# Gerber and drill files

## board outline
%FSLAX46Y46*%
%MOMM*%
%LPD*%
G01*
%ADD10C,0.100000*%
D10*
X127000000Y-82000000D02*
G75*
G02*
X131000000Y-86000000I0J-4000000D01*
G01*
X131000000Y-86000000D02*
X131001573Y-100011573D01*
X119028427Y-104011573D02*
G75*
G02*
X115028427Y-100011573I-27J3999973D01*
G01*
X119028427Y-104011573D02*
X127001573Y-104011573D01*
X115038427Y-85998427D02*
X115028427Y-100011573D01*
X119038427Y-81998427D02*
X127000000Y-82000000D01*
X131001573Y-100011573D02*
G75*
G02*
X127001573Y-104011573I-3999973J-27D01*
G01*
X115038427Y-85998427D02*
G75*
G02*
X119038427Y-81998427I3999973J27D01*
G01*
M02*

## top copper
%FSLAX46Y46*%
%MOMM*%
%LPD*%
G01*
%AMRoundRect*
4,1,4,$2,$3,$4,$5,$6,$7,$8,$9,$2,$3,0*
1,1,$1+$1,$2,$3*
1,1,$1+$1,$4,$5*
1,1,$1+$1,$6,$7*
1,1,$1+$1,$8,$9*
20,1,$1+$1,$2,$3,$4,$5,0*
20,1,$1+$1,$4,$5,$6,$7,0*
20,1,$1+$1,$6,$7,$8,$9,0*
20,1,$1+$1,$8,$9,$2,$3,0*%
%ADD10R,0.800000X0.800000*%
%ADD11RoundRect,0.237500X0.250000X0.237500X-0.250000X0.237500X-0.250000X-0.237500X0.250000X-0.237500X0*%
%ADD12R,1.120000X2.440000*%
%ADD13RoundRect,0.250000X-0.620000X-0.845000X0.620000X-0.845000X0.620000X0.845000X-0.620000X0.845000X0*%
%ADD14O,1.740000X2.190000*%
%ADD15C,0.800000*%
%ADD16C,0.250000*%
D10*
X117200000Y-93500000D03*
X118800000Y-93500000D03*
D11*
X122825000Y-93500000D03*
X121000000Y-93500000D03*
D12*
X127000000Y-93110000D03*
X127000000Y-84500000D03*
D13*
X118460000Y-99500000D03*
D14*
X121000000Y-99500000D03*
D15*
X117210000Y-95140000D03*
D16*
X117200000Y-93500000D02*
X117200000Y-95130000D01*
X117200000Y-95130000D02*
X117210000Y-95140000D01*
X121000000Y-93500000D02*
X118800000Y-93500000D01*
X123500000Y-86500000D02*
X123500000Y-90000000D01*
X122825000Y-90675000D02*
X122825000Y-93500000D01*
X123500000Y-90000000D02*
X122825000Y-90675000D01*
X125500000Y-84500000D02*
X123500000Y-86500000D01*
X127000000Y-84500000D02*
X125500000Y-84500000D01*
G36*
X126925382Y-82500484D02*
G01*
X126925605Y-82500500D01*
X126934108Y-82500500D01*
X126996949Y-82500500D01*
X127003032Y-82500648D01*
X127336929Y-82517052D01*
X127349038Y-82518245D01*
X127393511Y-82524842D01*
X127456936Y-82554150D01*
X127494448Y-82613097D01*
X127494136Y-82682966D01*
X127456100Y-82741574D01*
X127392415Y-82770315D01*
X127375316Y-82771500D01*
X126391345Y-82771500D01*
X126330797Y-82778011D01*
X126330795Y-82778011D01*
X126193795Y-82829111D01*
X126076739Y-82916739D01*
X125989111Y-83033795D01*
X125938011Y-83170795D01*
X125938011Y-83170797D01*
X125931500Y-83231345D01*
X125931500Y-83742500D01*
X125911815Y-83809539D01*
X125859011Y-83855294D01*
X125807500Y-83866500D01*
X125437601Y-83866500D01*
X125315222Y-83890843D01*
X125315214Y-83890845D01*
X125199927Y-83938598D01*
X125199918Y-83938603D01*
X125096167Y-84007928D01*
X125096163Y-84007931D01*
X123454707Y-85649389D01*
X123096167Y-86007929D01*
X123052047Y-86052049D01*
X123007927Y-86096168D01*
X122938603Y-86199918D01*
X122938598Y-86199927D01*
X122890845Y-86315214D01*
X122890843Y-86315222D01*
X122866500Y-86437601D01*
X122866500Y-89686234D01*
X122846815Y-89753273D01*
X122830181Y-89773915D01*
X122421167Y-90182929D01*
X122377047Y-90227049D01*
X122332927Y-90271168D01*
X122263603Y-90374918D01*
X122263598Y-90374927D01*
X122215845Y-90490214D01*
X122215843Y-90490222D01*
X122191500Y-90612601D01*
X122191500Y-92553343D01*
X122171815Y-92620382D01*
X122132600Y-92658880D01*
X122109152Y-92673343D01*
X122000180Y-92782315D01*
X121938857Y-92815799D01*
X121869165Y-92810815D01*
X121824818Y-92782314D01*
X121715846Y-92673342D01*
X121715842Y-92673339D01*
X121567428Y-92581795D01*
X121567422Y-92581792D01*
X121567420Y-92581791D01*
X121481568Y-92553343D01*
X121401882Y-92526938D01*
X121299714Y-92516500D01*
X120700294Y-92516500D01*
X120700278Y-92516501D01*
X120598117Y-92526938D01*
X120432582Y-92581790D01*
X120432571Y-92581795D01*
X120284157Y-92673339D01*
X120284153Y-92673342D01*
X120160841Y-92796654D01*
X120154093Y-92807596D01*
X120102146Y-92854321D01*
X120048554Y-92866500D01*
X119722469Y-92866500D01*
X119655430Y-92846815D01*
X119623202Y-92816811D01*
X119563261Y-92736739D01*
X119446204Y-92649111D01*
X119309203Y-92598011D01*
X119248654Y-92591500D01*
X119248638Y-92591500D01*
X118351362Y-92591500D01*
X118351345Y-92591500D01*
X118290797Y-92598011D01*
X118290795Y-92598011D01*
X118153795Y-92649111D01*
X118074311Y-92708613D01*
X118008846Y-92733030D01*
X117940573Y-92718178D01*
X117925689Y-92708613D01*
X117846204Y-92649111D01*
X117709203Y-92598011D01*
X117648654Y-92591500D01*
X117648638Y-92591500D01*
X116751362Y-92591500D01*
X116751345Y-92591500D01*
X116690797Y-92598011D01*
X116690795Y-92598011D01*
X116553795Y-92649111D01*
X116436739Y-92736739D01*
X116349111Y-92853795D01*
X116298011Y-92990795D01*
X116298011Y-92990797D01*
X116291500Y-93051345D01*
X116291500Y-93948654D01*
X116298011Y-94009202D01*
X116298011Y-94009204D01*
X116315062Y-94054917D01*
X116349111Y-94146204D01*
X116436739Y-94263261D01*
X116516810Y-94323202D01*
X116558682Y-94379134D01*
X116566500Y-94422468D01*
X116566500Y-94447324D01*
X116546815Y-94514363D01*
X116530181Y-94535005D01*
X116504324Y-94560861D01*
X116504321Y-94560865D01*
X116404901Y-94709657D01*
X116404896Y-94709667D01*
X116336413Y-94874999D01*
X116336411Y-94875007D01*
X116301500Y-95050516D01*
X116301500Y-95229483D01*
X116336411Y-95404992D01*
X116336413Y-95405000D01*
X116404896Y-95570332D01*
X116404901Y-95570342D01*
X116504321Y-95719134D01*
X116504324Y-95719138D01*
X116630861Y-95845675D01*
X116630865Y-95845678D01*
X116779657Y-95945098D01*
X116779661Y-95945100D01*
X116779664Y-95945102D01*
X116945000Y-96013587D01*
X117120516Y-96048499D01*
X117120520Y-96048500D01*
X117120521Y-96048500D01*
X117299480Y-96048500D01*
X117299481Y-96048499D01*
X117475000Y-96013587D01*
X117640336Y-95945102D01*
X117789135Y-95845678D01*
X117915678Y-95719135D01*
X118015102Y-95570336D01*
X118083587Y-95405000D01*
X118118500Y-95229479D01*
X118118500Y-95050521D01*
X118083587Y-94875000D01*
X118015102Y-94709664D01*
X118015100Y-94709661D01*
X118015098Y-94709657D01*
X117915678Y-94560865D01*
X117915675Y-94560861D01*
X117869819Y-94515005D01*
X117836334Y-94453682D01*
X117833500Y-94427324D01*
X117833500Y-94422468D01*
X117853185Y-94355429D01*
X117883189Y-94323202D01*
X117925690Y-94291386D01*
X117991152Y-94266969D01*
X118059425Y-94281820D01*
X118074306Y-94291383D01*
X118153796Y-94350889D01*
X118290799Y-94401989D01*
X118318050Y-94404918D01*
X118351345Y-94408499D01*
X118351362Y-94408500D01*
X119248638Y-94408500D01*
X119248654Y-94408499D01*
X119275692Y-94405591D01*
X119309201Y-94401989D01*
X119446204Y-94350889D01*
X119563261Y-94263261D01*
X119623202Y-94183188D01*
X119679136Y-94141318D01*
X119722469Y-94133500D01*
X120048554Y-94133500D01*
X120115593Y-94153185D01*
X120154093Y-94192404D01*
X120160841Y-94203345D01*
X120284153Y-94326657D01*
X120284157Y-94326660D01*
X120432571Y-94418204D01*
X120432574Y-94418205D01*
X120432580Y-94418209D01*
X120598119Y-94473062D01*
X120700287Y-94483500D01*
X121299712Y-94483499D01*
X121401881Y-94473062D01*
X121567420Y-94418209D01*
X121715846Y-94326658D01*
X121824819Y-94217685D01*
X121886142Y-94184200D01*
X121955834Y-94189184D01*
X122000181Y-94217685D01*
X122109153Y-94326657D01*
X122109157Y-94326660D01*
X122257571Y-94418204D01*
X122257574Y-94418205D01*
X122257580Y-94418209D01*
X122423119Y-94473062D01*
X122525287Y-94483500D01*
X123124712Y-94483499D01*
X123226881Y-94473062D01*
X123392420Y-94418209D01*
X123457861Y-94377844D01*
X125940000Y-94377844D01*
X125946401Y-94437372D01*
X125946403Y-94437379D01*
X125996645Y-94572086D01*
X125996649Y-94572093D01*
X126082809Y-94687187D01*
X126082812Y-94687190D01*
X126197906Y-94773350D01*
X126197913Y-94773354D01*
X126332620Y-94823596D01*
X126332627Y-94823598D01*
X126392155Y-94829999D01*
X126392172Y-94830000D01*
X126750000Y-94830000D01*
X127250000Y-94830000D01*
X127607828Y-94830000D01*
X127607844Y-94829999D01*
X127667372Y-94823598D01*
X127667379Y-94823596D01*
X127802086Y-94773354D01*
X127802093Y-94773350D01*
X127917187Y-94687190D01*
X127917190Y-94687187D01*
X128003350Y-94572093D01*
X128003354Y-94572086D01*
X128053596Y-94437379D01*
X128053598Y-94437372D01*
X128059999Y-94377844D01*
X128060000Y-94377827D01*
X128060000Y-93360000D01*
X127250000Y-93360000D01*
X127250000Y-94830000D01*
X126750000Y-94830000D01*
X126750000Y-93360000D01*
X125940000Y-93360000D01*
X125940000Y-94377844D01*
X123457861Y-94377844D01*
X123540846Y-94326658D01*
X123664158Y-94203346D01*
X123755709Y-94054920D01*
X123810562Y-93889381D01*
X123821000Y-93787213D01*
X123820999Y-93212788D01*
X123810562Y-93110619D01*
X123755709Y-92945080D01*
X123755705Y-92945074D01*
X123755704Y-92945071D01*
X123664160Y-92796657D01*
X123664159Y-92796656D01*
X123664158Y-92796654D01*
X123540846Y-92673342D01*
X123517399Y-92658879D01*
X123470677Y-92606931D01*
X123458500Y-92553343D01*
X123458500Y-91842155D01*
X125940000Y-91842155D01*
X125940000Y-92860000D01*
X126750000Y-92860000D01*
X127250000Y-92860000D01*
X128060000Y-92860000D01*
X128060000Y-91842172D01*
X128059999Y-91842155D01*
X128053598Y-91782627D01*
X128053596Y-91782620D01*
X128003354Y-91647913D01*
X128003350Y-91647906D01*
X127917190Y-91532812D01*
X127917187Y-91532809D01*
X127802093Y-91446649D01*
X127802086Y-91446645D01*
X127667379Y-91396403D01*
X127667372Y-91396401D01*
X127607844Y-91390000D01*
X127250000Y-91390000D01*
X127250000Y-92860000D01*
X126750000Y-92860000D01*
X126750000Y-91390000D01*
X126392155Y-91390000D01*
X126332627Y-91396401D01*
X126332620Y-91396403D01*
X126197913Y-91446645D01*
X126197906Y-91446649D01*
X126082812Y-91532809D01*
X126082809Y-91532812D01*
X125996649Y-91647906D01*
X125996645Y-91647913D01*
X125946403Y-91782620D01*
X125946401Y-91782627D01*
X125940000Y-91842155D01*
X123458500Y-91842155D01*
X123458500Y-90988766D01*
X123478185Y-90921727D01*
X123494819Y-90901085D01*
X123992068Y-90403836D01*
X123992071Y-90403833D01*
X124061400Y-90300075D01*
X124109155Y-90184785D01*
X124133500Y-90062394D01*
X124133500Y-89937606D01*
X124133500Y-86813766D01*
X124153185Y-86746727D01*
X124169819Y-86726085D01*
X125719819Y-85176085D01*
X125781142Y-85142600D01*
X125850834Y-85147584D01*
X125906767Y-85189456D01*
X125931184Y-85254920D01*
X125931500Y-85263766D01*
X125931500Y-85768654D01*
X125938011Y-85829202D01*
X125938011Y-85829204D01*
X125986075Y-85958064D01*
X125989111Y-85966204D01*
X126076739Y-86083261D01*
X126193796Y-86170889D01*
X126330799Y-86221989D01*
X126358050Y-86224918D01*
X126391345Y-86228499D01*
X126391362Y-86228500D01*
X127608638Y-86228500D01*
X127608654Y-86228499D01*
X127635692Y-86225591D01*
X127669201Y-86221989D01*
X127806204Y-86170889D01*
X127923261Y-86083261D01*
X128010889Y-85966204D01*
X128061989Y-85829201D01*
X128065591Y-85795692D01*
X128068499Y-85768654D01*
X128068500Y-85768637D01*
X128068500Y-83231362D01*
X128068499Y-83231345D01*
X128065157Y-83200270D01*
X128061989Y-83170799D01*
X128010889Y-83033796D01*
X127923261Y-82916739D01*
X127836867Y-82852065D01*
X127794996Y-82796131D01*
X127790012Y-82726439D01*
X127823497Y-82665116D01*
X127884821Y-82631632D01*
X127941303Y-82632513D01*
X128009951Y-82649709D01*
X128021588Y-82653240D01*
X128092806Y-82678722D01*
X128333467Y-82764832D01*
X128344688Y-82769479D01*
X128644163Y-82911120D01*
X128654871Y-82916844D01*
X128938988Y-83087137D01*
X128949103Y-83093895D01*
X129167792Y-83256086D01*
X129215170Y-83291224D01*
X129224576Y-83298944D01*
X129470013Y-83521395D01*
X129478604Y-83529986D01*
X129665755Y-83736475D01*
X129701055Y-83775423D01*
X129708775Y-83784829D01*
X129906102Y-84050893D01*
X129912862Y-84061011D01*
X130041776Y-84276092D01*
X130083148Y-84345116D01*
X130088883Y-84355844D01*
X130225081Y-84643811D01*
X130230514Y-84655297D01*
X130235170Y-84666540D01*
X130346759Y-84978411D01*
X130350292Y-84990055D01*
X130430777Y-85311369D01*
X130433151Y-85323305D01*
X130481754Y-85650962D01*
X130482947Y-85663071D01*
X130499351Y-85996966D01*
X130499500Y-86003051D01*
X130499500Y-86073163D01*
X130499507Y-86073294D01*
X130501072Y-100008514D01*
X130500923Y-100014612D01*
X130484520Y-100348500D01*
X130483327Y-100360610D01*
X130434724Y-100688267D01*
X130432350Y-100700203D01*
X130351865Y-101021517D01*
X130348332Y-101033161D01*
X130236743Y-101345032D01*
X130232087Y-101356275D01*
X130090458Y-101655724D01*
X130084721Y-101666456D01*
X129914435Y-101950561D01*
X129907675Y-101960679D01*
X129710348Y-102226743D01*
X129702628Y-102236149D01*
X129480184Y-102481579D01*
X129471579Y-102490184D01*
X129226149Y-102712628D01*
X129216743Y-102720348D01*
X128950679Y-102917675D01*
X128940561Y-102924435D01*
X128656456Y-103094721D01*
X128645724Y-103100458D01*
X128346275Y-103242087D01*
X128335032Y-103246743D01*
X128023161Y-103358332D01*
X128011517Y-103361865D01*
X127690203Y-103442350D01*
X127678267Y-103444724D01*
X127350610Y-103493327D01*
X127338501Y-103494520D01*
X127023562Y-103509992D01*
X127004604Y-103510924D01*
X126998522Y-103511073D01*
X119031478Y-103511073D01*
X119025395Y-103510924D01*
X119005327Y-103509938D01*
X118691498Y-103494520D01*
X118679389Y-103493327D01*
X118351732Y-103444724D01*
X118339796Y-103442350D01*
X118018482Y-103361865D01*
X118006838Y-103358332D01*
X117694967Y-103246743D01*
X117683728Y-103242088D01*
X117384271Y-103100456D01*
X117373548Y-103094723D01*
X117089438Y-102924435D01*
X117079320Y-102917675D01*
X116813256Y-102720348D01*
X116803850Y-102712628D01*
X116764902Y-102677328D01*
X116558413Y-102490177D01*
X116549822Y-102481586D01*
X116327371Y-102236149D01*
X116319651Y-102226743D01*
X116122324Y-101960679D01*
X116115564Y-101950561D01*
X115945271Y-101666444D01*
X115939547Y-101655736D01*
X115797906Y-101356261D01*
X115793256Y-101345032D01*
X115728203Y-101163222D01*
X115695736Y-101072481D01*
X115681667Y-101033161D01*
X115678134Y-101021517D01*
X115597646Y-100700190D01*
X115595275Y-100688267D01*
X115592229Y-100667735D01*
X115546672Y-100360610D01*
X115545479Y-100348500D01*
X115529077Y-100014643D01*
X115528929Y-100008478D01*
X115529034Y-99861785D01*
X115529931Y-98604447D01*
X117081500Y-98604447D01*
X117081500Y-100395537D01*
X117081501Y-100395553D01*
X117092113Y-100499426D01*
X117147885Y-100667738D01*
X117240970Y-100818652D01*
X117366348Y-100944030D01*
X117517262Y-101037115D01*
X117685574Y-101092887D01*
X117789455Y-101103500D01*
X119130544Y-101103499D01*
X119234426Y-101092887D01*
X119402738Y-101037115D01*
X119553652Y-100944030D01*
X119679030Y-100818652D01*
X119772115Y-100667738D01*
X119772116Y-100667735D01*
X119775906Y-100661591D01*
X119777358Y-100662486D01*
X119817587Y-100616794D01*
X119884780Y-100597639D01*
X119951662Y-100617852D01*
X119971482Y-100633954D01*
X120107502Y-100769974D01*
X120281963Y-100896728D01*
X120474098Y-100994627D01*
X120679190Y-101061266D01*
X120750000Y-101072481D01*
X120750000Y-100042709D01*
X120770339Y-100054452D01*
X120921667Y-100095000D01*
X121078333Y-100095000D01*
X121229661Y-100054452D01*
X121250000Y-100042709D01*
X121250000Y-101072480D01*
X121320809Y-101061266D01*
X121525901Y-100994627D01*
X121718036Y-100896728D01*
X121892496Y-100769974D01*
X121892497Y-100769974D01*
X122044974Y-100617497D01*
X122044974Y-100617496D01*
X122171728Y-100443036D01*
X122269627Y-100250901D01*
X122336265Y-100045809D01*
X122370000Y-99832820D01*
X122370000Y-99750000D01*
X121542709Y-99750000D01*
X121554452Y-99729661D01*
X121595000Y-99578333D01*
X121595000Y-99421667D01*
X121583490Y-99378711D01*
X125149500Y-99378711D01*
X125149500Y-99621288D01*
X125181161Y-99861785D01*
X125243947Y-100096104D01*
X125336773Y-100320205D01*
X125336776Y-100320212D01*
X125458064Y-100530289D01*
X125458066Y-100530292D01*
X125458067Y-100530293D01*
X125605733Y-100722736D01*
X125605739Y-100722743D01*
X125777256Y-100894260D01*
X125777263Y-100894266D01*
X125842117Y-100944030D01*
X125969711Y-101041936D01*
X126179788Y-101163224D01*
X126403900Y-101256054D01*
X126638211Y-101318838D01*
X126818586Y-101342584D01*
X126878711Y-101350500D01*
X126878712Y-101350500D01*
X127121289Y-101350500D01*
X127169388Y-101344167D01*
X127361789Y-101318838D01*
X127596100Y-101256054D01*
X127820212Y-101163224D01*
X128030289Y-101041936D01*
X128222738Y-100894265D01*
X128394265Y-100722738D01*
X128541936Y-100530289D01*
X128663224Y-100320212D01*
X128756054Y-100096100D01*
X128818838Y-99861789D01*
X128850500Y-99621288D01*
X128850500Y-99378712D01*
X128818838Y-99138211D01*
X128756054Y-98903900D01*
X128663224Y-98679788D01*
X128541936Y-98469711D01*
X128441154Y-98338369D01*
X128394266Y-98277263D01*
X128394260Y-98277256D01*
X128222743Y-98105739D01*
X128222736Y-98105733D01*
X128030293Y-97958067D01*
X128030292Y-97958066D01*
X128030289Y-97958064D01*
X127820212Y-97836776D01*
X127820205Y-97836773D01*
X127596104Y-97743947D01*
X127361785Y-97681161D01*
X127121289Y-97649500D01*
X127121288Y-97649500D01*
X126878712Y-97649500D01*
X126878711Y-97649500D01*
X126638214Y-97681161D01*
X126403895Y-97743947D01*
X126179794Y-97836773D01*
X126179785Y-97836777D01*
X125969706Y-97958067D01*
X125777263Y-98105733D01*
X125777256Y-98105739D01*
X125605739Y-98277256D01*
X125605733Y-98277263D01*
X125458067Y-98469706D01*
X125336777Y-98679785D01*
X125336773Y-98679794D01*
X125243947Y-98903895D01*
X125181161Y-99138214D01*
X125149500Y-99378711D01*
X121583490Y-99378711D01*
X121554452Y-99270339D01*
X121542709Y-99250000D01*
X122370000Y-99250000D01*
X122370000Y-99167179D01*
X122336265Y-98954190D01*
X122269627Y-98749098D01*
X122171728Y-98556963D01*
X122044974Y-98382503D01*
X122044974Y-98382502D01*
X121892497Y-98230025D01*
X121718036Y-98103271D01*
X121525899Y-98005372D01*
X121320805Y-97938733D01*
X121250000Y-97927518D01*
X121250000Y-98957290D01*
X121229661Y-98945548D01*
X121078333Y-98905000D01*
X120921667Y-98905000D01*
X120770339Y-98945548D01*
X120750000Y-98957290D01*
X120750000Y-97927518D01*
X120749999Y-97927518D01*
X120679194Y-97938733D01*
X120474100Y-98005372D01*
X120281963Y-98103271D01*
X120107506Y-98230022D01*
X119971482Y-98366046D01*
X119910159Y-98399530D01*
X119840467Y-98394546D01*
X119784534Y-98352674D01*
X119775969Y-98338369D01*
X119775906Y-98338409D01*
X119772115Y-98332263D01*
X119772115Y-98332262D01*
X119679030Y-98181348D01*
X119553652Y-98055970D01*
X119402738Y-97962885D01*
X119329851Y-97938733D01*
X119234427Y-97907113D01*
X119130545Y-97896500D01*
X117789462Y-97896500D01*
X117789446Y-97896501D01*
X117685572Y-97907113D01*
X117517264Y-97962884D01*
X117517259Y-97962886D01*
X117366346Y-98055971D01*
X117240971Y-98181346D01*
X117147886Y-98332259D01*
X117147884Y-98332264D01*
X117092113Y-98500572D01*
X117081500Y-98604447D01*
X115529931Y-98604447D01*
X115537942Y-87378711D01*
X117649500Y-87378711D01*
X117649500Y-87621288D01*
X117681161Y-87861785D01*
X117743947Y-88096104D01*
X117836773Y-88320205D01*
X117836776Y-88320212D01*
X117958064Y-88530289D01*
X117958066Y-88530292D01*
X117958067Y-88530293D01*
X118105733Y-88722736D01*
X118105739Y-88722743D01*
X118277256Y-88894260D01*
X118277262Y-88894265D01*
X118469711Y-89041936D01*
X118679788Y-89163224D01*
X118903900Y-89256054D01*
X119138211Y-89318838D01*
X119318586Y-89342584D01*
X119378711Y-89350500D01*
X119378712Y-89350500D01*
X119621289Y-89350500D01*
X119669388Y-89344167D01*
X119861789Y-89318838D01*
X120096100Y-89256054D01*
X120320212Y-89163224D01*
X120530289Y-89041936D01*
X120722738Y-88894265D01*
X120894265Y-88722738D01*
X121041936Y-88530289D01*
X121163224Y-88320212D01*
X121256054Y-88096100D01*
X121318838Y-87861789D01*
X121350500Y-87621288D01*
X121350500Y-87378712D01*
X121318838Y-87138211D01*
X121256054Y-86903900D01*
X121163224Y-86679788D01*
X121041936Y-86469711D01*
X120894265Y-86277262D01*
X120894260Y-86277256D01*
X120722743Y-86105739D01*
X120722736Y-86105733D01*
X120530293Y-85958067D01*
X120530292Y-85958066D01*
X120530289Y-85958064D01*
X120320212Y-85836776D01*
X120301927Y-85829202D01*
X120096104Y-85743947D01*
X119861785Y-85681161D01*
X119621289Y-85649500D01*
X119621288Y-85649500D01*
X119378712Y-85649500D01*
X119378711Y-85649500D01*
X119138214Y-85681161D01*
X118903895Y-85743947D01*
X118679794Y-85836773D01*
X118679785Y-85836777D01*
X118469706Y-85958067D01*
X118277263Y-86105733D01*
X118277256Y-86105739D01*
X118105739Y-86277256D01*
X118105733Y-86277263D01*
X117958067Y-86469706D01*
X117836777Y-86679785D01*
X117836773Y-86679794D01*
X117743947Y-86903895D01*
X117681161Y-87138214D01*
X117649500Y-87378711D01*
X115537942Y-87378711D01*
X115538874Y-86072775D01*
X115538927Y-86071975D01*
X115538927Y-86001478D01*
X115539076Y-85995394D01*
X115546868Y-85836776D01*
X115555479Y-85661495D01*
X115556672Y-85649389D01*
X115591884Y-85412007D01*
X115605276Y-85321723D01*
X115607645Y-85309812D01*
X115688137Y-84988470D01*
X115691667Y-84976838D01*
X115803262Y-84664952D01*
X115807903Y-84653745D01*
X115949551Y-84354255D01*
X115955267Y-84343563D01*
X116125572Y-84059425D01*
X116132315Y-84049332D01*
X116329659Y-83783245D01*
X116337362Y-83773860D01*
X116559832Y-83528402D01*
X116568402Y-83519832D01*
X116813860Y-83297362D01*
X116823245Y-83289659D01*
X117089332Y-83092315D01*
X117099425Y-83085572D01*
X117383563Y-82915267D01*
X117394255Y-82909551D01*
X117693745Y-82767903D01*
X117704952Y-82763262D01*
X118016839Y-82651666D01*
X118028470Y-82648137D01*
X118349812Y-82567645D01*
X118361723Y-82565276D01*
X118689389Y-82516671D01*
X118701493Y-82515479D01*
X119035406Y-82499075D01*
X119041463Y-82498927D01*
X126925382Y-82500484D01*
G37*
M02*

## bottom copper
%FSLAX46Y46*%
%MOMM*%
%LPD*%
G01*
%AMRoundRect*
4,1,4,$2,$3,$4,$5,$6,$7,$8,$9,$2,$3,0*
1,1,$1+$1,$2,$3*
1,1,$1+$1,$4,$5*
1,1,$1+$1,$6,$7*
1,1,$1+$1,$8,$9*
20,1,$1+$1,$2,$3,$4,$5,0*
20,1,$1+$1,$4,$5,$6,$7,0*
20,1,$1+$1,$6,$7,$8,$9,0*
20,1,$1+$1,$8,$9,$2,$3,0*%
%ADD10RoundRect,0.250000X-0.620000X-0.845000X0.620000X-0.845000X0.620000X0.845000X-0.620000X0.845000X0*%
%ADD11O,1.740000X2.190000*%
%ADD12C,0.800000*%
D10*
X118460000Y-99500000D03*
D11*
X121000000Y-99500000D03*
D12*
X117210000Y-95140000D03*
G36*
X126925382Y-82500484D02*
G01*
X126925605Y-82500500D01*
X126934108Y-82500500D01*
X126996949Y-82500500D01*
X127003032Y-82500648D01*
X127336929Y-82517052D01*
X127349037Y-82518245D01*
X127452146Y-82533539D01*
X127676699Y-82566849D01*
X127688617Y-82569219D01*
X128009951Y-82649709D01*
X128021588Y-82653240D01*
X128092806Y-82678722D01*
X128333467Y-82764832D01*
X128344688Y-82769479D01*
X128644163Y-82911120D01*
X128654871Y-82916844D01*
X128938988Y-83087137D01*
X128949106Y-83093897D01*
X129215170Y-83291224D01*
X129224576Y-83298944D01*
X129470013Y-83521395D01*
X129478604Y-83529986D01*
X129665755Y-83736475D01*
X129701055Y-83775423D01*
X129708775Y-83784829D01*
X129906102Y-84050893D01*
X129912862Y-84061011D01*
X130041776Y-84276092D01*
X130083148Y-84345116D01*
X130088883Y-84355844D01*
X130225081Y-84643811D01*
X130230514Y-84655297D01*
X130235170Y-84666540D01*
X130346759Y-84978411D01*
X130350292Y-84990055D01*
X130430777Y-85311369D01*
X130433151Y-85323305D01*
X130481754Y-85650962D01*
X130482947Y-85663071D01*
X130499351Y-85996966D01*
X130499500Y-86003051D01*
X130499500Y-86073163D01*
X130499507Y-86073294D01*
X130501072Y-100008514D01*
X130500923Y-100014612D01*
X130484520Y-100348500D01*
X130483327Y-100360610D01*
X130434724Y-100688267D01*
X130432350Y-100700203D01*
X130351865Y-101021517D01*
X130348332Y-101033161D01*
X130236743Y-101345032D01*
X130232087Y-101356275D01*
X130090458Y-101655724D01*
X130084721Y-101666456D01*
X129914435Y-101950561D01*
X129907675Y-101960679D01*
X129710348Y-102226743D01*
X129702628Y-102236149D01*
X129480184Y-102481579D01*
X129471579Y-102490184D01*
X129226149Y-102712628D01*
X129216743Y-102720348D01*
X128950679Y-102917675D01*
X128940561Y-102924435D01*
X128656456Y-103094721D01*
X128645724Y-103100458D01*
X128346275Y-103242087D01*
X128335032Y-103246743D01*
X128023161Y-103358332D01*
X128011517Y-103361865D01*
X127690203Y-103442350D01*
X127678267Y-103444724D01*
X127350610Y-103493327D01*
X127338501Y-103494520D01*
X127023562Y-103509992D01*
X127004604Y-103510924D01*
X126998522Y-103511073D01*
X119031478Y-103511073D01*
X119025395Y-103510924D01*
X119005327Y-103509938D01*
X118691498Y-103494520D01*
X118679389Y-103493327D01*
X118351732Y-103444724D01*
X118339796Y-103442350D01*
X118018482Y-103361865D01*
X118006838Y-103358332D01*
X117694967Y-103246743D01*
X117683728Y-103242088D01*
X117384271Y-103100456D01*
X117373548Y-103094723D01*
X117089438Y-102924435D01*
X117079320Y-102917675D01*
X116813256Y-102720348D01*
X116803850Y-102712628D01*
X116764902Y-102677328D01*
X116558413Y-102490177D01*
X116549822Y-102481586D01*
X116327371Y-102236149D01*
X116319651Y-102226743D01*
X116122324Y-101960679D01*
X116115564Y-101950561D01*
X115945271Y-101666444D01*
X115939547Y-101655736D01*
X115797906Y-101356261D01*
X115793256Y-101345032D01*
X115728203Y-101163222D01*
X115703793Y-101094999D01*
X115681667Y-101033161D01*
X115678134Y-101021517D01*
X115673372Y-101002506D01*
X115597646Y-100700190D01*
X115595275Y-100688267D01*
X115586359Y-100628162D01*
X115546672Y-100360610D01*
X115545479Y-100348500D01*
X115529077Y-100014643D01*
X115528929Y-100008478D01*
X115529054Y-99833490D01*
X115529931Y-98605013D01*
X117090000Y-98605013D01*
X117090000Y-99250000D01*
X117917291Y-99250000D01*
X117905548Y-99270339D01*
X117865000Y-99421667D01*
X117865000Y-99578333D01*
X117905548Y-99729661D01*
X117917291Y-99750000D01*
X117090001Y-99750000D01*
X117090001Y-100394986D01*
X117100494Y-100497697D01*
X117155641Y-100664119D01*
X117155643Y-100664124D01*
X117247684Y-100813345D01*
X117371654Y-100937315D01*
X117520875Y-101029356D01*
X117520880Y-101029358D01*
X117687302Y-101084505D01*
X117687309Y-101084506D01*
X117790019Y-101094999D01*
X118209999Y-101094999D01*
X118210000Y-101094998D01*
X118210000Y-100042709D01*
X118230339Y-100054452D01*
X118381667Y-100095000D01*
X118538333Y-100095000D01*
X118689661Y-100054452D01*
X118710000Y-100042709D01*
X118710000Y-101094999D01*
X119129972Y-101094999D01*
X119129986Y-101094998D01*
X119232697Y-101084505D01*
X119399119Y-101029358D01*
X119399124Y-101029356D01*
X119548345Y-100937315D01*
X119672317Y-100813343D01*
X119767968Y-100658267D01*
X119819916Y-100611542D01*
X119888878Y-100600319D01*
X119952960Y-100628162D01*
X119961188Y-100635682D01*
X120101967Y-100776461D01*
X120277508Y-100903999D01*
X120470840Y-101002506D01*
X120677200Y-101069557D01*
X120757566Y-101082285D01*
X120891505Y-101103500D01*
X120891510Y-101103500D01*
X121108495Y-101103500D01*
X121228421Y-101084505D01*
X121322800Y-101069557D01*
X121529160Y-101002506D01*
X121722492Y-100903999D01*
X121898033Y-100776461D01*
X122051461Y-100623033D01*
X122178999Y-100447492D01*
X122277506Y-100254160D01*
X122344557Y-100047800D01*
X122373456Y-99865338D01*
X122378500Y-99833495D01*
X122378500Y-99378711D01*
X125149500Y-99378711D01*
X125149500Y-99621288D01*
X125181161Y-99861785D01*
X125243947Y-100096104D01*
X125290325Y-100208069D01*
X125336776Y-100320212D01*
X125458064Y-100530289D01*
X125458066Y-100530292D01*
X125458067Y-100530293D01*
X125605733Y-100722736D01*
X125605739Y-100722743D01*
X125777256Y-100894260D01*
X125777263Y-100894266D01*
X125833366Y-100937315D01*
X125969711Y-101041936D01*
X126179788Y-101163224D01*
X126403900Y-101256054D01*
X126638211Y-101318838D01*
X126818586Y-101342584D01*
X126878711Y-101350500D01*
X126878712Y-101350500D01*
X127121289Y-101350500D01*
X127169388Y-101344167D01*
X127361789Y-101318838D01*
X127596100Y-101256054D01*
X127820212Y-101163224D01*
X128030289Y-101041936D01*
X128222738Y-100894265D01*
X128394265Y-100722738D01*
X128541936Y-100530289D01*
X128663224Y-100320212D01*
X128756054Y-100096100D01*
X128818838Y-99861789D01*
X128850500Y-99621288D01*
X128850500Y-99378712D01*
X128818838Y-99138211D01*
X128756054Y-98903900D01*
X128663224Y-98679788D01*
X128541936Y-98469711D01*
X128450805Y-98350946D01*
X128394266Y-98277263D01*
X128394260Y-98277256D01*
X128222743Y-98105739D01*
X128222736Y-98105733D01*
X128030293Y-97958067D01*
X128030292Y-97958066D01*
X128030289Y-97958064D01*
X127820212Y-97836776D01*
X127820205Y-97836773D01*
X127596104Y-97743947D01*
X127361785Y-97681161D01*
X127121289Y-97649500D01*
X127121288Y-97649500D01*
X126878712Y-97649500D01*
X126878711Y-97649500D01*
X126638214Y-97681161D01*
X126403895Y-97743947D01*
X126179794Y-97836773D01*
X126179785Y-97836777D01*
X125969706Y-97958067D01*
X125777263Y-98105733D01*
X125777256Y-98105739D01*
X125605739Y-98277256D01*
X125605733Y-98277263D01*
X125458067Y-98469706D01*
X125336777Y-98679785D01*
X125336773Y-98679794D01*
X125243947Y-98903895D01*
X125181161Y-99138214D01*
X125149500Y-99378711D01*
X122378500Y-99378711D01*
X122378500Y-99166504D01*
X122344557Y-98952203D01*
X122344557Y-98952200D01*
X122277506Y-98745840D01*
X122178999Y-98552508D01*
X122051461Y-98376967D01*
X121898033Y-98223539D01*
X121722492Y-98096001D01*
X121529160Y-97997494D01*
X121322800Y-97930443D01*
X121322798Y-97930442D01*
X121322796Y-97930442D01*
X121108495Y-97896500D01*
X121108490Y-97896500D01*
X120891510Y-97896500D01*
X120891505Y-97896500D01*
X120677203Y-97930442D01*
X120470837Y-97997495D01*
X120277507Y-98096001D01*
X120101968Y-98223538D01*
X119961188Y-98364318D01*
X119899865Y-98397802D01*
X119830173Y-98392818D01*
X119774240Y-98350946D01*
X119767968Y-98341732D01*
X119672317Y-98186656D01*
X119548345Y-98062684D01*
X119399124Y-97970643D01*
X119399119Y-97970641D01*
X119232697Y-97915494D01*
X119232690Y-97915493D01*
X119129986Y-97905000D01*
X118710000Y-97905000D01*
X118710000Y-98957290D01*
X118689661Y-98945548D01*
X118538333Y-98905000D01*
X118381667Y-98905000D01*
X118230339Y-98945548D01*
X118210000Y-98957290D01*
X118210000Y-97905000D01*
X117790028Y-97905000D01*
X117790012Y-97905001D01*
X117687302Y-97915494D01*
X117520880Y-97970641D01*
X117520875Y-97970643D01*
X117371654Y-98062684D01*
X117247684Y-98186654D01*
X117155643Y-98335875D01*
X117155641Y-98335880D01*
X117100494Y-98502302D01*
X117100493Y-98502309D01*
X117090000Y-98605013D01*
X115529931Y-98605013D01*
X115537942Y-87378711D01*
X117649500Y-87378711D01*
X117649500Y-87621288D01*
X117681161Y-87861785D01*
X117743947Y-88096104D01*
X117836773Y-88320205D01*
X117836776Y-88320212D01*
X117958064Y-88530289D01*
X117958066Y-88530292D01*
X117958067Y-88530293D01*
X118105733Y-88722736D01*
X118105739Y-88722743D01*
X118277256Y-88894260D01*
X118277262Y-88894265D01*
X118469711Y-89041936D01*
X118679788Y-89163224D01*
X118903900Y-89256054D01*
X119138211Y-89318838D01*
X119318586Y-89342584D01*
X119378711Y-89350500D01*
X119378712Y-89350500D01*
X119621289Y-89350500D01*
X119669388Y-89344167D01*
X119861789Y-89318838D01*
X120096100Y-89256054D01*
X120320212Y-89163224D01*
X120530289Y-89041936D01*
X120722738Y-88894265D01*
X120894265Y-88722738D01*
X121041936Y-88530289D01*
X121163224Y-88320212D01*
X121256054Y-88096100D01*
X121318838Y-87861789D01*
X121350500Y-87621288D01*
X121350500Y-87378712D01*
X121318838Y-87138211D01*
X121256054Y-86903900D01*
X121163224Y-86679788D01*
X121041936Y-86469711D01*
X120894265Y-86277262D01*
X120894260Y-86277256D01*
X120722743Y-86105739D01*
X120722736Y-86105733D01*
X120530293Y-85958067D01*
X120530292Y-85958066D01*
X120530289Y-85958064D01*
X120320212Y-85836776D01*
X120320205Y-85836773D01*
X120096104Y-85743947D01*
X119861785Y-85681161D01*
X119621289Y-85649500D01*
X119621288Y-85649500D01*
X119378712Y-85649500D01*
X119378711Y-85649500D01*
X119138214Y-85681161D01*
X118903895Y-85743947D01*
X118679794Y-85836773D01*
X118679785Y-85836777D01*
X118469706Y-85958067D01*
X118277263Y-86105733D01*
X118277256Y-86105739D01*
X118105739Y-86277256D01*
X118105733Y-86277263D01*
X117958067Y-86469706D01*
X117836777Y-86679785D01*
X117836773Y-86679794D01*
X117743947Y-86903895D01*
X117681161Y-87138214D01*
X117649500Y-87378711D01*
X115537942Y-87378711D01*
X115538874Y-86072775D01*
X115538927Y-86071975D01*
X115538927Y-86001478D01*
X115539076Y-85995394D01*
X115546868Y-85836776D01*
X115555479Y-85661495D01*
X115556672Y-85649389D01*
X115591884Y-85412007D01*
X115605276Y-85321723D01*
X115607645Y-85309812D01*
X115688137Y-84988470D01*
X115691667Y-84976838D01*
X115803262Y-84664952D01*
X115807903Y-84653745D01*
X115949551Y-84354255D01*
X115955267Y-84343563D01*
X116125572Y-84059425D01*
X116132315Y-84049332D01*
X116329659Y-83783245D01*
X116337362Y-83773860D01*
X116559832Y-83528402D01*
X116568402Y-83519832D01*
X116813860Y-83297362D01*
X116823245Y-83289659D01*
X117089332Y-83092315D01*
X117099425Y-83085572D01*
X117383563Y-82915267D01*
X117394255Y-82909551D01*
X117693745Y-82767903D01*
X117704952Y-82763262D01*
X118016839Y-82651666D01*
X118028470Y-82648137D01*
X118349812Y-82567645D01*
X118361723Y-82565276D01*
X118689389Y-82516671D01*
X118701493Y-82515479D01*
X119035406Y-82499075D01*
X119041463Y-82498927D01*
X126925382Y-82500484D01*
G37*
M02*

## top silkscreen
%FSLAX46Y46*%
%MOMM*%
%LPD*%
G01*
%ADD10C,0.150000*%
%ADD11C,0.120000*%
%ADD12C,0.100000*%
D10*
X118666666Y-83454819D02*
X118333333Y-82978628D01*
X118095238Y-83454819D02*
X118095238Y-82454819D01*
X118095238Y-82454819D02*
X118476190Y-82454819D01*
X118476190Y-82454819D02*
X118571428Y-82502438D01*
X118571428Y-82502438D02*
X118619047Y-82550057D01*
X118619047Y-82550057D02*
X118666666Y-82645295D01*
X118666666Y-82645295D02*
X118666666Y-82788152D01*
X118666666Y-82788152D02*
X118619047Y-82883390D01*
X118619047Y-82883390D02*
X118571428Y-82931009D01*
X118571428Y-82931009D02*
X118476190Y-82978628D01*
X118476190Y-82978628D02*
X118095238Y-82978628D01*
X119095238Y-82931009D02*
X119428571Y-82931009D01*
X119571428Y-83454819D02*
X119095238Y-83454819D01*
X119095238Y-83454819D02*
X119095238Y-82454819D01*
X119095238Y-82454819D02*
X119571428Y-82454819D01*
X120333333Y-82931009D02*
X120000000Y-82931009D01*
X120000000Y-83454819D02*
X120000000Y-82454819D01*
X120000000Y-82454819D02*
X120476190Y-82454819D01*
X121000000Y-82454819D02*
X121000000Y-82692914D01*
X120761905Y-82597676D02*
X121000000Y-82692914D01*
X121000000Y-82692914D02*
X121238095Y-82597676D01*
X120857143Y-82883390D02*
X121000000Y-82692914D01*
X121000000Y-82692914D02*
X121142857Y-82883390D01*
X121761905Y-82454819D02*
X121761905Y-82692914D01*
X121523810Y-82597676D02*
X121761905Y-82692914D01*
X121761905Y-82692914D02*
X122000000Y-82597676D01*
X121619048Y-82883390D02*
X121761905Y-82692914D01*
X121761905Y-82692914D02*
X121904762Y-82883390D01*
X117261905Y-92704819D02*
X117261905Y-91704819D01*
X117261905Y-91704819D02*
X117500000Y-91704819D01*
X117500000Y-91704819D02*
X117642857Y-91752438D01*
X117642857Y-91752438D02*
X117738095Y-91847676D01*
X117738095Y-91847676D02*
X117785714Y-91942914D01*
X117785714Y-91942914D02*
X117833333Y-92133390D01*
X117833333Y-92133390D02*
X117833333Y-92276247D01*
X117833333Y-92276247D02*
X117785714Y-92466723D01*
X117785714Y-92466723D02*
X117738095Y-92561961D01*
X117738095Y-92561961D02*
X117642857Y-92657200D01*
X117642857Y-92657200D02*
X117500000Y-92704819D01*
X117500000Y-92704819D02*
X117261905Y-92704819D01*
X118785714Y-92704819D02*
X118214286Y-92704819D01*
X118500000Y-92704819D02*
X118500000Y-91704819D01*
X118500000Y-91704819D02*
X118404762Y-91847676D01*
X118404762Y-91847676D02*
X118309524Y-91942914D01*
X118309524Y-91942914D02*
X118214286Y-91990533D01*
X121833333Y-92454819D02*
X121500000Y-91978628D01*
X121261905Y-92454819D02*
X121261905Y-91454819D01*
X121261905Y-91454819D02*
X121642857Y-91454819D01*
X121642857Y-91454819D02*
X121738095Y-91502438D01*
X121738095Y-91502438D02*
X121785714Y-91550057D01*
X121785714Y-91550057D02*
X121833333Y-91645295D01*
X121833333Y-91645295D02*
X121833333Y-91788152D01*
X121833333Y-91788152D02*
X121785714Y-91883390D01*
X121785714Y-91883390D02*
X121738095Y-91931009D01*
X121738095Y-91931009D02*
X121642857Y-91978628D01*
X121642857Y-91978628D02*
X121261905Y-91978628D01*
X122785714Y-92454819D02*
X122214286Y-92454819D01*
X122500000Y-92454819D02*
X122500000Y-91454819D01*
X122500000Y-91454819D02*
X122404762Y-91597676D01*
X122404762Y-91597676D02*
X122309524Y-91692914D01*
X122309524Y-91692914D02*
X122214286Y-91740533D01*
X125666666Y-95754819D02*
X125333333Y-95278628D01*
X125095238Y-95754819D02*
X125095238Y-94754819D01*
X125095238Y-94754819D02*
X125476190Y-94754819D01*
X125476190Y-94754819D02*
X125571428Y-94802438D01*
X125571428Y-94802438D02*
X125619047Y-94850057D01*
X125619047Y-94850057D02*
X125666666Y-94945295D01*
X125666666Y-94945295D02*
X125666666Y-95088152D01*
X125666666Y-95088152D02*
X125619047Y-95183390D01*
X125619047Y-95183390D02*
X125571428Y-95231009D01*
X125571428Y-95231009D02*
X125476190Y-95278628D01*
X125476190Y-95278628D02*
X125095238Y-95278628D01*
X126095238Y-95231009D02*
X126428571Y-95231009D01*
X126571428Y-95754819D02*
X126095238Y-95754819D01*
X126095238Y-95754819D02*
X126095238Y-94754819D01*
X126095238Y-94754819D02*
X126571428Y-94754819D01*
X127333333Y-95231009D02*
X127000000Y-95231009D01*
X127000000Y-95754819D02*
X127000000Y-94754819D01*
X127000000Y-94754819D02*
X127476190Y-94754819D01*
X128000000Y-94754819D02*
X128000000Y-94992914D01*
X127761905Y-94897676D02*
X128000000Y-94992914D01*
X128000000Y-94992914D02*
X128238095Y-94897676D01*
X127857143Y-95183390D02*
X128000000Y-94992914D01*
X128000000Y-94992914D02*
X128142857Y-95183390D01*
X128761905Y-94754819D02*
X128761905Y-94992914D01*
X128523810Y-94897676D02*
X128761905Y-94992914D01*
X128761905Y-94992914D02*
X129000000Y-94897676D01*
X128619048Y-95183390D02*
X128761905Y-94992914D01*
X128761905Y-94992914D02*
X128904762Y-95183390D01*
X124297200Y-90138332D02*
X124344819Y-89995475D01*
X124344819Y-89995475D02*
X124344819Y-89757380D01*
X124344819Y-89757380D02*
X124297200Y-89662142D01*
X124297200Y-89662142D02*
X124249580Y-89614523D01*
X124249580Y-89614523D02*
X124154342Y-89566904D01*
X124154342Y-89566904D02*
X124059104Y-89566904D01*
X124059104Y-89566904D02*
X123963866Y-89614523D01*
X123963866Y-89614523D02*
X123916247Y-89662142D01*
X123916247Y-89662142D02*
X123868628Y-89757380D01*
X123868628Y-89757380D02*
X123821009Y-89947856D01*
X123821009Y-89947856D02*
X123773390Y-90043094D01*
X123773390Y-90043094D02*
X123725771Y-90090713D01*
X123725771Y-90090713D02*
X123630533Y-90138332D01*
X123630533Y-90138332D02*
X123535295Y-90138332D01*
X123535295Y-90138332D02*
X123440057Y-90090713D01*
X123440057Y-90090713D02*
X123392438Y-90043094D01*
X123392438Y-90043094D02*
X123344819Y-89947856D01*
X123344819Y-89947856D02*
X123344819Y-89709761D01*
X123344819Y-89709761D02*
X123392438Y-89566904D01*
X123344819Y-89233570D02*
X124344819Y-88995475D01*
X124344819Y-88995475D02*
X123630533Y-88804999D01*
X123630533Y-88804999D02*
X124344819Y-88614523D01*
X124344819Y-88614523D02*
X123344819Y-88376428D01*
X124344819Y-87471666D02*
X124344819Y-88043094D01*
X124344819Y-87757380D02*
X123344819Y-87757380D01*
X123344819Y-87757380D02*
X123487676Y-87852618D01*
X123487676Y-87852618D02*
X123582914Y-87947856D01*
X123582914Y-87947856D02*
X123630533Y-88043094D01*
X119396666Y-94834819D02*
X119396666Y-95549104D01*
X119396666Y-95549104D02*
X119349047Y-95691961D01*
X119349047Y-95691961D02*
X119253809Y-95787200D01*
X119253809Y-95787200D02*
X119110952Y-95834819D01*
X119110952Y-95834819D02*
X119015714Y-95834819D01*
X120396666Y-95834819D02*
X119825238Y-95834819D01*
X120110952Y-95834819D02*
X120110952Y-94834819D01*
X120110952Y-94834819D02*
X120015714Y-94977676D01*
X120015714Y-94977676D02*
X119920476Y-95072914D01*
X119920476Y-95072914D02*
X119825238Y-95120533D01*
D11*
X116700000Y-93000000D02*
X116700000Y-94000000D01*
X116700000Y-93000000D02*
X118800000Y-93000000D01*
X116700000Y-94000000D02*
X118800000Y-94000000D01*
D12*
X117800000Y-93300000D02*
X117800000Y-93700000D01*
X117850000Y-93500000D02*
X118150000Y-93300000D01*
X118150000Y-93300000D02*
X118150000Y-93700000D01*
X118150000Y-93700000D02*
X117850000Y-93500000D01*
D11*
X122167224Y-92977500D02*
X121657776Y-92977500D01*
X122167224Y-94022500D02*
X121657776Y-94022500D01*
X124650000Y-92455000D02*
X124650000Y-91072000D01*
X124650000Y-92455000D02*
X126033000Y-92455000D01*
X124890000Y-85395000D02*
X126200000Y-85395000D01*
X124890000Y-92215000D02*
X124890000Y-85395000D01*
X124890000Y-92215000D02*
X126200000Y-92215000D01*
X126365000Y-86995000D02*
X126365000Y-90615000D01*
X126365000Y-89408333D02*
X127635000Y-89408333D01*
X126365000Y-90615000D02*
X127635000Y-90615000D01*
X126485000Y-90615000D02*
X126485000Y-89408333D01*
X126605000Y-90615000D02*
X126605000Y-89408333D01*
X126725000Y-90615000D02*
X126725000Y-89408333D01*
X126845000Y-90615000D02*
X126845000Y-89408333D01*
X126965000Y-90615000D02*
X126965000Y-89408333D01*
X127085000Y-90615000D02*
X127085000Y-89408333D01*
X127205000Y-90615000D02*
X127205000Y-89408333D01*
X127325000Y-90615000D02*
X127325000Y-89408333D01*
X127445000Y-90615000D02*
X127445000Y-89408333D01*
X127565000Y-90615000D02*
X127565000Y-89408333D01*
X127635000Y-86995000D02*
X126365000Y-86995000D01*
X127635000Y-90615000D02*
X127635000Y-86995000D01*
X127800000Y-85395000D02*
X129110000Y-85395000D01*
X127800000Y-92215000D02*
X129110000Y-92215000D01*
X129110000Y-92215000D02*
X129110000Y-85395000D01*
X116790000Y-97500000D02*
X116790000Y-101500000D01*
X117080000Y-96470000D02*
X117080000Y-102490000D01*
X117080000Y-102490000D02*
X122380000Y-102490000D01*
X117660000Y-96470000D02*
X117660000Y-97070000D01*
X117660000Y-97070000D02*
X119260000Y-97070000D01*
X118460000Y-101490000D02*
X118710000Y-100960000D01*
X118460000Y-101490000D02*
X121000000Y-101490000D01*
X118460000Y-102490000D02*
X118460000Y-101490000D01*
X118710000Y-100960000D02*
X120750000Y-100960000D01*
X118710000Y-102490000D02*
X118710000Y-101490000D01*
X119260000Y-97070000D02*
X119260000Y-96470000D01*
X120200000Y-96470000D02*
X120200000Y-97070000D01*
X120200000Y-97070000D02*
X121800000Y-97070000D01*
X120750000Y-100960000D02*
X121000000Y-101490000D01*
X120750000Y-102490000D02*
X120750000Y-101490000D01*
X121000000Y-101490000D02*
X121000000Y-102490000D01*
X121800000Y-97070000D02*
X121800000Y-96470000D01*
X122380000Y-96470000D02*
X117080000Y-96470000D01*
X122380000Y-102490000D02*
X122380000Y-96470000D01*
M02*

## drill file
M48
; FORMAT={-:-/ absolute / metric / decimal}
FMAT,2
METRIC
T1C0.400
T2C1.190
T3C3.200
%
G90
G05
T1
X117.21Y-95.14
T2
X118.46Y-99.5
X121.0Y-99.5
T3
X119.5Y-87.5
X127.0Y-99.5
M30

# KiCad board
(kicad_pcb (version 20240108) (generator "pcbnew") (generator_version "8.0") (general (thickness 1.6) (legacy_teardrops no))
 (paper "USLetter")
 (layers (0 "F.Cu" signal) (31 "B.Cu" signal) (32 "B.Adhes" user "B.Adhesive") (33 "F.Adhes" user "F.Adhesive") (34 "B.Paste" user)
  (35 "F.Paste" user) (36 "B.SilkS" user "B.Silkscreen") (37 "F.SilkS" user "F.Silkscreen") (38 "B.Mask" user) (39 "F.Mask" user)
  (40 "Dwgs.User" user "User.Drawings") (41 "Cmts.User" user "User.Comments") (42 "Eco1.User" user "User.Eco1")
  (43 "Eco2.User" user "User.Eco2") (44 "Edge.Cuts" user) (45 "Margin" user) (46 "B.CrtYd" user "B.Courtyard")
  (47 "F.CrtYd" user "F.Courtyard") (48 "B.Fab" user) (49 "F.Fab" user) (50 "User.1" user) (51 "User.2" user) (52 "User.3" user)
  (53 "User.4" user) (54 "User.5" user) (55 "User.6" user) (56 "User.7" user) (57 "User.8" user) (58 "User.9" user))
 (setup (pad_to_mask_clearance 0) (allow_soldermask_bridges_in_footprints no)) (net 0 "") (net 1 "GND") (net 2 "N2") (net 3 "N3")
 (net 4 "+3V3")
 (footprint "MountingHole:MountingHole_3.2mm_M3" (layer "F.Cu") (at 119.5 87.5)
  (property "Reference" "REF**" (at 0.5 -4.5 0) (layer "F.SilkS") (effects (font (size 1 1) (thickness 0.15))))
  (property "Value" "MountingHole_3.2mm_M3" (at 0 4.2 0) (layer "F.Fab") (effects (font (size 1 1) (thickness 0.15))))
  (pad "" np_thru_hole circle (at 0 0) (size 3.2 3.2) (drill 3.2) (layers "*.Cu" "*.Mask")))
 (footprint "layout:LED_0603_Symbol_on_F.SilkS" (layer "F.Cu") (at 118 93.5)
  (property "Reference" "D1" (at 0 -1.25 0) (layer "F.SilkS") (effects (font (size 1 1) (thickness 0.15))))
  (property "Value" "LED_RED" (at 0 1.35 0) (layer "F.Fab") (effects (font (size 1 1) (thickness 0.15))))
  (fp_line (start -1.3 -0.5) (end -1.3 0.5) (stroke (width 0.12) (type solid)) (layer "F.SilkS"))
  (fp_line (start -1.3 -0.5) (end 0.8 -0.5) (stroke (width 0.12) (type solid)) (layer "F.SilkS"))
  (fp_line (start -1.3 0.5) (end 0.8 0.5) (stroke (width 0.12) (type solid)) (layer "F.SilkS"))
  (fp_line (start -0.2 -0.2) (end -0.2 0.2) (stroke (width 0.1) (type solid)) (layer "F.SilkS"))
  (fp_line (start -0.15 0) (end 0.15 -0.2) (stroke (width 0.1) (type solid)) (layer "F.SilkS"))
  (fp_line (start 0.15 -0.2) (end 0.15 0.2) (stroke (width 0.1) (type solid)) (layer "F.SilkS"))
  (fp_line (start 0.15 0.2) (end -0.15 0) (stroke (width 0.1) (type solid)) (layer "F.SilkS"))
  (pad "1" smd rect (at -0.8 0 180) (size 0.8 0.8) (layers "F.Cu" "F.Paste" "F.Mask") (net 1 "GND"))
  (pad "2" smd rect (at 0.8 0 180) (size 0.8 0.8) (layers "F.Cu" "F.Paste" "F.Mask") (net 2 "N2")))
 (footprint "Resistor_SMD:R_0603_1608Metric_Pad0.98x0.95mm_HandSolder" (layer "F.Cu") (at 121.9125 93.5 180)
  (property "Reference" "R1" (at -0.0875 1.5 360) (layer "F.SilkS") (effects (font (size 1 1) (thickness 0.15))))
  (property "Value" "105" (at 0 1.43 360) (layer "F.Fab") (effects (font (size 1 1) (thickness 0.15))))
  (fp_line (start -0.254724 0.5225) (end 0.254724 0.5225) (stroke (width 0.12) (type solid)) (layer "F.SilkS"))
  (fp_line (start -0.254724 -0.5225) (end 0.254724 -0.5225) (stroke (width 0.12) (type solid)) (layer "F.SilkS"))
  (pad "1" smd roundrect (at -0.9125 0 180) (size 0.975 0.95) (layers "F.Cu" "F.Paste" "F.Mask") (roundrect_rratio 0.25) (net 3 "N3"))
  (pad "2" smd roundrect (at 0.9125 0 180) (size 0.975 0.95) (layers "F.Cu" "F.Paste" "F.Mask") (roundrect_rratio 0.25) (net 2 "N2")))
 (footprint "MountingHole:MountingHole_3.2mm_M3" (layer "F.Cu") (at 127 99.5)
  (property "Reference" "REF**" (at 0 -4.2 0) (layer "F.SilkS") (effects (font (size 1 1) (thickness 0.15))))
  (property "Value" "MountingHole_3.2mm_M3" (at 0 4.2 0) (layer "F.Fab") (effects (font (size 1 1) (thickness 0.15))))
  (pad "" np_thru_hole circle (at 0 0) (size 3.2 3.2) (drill 3.2) (layers "*.Cu" "*.Mask")))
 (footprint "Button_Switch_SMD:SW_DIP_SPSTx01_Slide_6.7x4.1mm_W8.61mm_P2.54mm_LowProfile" (layer "F.Cu") (at 127 88.805 90)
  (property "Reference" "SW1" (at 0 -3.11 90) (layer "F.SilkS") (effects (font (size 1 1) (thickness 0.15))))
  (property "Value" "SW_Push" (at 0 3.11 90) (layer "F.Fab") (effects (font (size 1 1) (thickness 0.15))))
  (fp_line (start -3.65 -2.35) (end -2.267 -2.35) (stroke (width 0.12) (type solid)) (layer "F.SilkS"))
  (fp_line (start -3.65 -2.35) (end -3.65 -0.967) (stroke (width 0.12) (type solid)) (layer "F.SilkS"))
  (fp_line (start 3.41 -2.11) (end 3.41 -0.8) (stroke (width 0.12) (type solid)) (layer "F.SilkS"))
  (fp_line (start -3.41 -2.11) (end 3.41 -2.11) (stroke (width 0.12) (type solid)) (layer "F.SilkS"))
  (fp_line (start -3.41 -2.11) (end -3.41 -0.8) (stroke (width 0.12) (type solid)) (layer "F.SilkS"))
  (fp_line (start 1.81 -0.635) (end -1.81 -0.635) (stroke (width 0.12) (type solid)) (layer "F.SilkS"))
  (fp_line (start -0.603333 -0.635) (end -0.603333 0.635) (stroke (width 0.12) (type solid)) (layer "F.SilkS"))
  (fp_line (start -1.81 -0.635) (end -1.81 0.635) (stroke (width 0.12) (type solid)) (layer "F.SilkS"))
  (fp_line (start -1.81 -0.515) (end -0.603333 -0.515) (stroke (width 0.12) (type solid)) (layer "F.SilkS"))
  (fp_line (start -1.81 -0.395) (end -0.603333 -0.395) (stroke (width 0.12) (type solid)) (layer "F.SilkS"))
  (fp_line (start -1.81 -0.275) (end -0.603333 -0.275) (stroke (width 0.12) (type solid)) (layer "F.SilkS"))
  (fp_line (start -1.81 -0.155) (end -0.603333 -0.155) (stroke (width 0.12) (type solid)) (layer "F.SilkS"))
  (fp_line (start -1.81 -0.035) (end -0.603333 -0.035) (stroke (width 0.12) (type solid)) (layer "F.SilkS"))
  (fp_line (start -1.81 0.085) (end -0.603333 0.085) (stroke (width 0.12) (type solid)) (layer "F.SilkS"))
  (fp_line (start -1.81 0.205) (end -0.603333 0.205) (stroke (width 0.12) (type solid)) (layer "F.SilkS"))
  (fp_line (start -1.81 0.325) (end -0.603333 0.325) (stroke (width 0.12) (type solid)) (layer "F.SilkS"))
  (fp_line (start -1.81 0.445) (end -0.603333 0.445) (stroke (width 0.12) (type solid)) (layer "F.SilkS"))
  (fp_line (start -1.81 0.565) (end -0.603333 0.565) (stroke (width 0.12) (type solid)) (layer "F.SilkS"))
  (fp_line (start 1.81 0.635) (end 1.81 -0.635) (stroke (width 0.12) (type solid)) (layer "F.SilkS"))
  (fp_line (start -1.81 0.635) (end 1.81 0.635) (stroke (width 0.12) (type solid)) (layer "F.SilkS"))
  (fp_line (start 3.41 0.8) (end 3.41 2.11) (stroke (width 0.12) (type solid)) (layer "F.SilkS"))
  (fp_line (start -3.41 0.8) (end -3.41 2.11) (stroke (width 0.12) (type solid)) (layer "F.SilkS"))
  (fp_line (start -3.41 2.11) (end 3.41 2.11) (stroke (width 0.12) (type solid)) (layer "F.SilkS"))
  (pad "1" smd rect (at -4.305 0 90) (size 2.44 1.12) (layers "F.Cu" "F.Paste" "F.Mask") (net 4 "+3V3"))
  (pad "2" smd rect (at 4.305 0 90) (size 2.44 1.12) (layers "F.Cu" "F.Paste" "F.Mask") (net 3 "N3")))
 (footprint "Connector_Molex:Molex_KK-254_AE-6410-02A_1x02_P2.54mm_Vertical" (layer "F.Cu") (at 118.46 99.5)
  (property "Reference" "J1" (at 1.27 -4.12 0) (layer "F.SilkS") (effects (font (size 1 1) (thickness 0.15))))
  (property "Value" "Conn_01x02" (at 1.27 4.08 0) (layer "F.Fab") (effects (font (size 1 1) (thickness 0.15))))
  (fp_line (start -1.67 -2) (end -1.67 2) (stroke (width 0.12) (type solid)) (layer "F.SilkS"))
  (fp_line (start -1.38 -3.03) (end -1.38 2.99) (stroke (width 0.12) (type solid)) (layer "F.SilkS"))
  (fp_line (start -1.38 2.99) (end 3.92 2.99) (stroke (width 0.12) (type solid)) (layer "F.SilkS"))
  (fp_line (start -0.8 -3.03) (end -0.8 -2.43) (stroke (width 0.12) (type solid)) (layer "F.SilkS"))
  (fp_line (start -0.8 -2.43) (end 0.8 -2.43) (stroke (width 0.12) (type solid)) (layer "F.SilkS"))
  (fp_line (start 0 1.99) (end 0.25 1.46) (stroke (width 0.12) (type solid)) (layer "F.SilkS"))
  (fp_line (start 0 1.99) (end 2.54 1.99) (stroke (width 0.12) (type solid)) (layer "F.SilkS"))
  (fp_line (start 0 2.99) (end 0 1.99) (stroke (width 0.12) (type solid)) (layer "F.SilkS"))
  (fp_line (start 0.25 1.46) (end 2.29 1.46) (stroke (width 0.12) (type solid)) (layer "F.SilkS"))
  (fp_line (start 0.25 2.99) (end 0.25 1.99) (stroke (width 0.12) (type solid)) (layer "F.SilkS"))
  (fp_line (start 0.8 -2.43) (end 0.8 -3.03) (stroke (width 0.12) (type solid)) (layer "F.SilkS"))
  (fp_line (start 1.74 -3.03) (end 1.74 -2.43) (stroke (width 0.12) (type solid)) (layer "F.SilkS"))
  (fp_line (start 1.74 -2.43) (end 3.34 -2.43) (stroke (width 0.12) (type solid)) (layer "F.SilkS"))
  (fp_line (start 2.29 1.46) (end 2.54 1.99) (stroke (width 0.12) (type solid)) (layer "F.SilkS"))
  (fp_line (start 2.29 2.99) (end 2.29 1.99) (stroke (width 0.12) (type solid)) (layer "F.SilkS"))
  (fp_line (start 2.54 1.99) (end 2.54 2.99) (stroke (width 0.12) (type solid)) (layer "F.SilkS"))
  (fp_line (start 3.34 -2.43) (end 3.34 -3.03) (stroke (width 0.12) (type solid)) (layer "F.SilkS"))
  (fp_line (start 3.92 -3.03) (end -1.38 -3.03) (stroke (width 0.12) (type solid)) (layer "F.SilkS"))
  (fp_line (start 3.92 2.99) (end 3.92 -3.03) (stroke (width 0.12) (type solid)) (layer "F.SilkS"))
  (pad "1" thru_hole roundrect (at 0 0) (size 1.74 2.19) (drill 1.19) (layers "*.Cu" "*.Mask") (remove_unused_layers no)
   (roundrect_rratio 0.143678) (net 1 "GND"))
  (pad "2" thru_hole oval (at 2.54 0) (size 1.74 2.19) (drill 1.19) (layers "*.Cu" "*.Mask") (remove_unused_layers no) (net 4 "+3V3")))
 (gr_arc (start 127 82) (mid 129.828427 83.171573) (end 131 86) (stroke (width 0.1) (type default)) (layer "Edge.Cuts"))
 (gr_line (start 131 86) (end 131.001573 100.011573) (stroke (width 0.1) (type default)) (layer "Edge.Cuts"))
 (gr_arc (start 119.028427 104.011573) (mid 116.2 102.84) (end 115.028427 100.011573) (stroke (width 0.1) (type default))
  (layer "Edge.Cuts"))
 (gr_line (start 119.028427 104.011573) (end 127.001573 104.011573) (stroke (width 0.1) (type default)) (layer "Edge.Cuts"))
 (gr_line (start 115.038427 85.998427) (end 115.028427 100.011573) (stroke (width 0.1) (type default)) (layer "Edge.Cuts"))
 (gr_line (start 119.038427 81.998427) (end 127 82) (stroke (width 0.1) (type default)) (layer "Edge.Cuts"))
 (gr_arc (start 131.001573 100.011573) (mid 129.83 102.84) (end 127.001573 104.011573) (stroke (width 0.1) (type default))
  (layer "Edge.Cuts"))
 (gr_arc (start 115.038427 85.998427) (mid 116.21 83.17) (end 119.038427 81.998427) (stroke (width 0.1) (type default)) (layer "Edge.Cuts"))
 (segment (start 117.2 93.5) (end 117.2 95.13) (width 0.25) (layer "F.Cu") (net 1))
 (segment (start 117.2 95.13) (end 117.21 95.14) (width 0.25) (layer "F.Cu") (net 1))
 (via (at 117.21 95.14) (size 0.8) (drill 0.4) (layers "F.Cu" "B.Cu") (free yes) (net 1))
 (segment (start 121 93.5) (end 118.8 93.5) (width 0.25) (layer "F.Cu") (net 2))
 (segment (start 123.5 86.5) (end 123.5 90) (width 0.25) (layer "F.Cu") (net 3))
 (segment (start 122.825 90.675) (end 122.825 93.5) (width 0.25) (layer "F.Cu") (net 3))
 (segment (start 123.5 90) (end 122.825 90.675) (width 0.25) (layer "F.Cu") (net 3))
 (segment (start 125.5 84.5) (end 123.5 86.5) (width 0.25) (layer "F.Cu") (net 3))
 (segment (start 127 84.5) (end 125.5 84.5) (width 0.25) (layer "F.Cu") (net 3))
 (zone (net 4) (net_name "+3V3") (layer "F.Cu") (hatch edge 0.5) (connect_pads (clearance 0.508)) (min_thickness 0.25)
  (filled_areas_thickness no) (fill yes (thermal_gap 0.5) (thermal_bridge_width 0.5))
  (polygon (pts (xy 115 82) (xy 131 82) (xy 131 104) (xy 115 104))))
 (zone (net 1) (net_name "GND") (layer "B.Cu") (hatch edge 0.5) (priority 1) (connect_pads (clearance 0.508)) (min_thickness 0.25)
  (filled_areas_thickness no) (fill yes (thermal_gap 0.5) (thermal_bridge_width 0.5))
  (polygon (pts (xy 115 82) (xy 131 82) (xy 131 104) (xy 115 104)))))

